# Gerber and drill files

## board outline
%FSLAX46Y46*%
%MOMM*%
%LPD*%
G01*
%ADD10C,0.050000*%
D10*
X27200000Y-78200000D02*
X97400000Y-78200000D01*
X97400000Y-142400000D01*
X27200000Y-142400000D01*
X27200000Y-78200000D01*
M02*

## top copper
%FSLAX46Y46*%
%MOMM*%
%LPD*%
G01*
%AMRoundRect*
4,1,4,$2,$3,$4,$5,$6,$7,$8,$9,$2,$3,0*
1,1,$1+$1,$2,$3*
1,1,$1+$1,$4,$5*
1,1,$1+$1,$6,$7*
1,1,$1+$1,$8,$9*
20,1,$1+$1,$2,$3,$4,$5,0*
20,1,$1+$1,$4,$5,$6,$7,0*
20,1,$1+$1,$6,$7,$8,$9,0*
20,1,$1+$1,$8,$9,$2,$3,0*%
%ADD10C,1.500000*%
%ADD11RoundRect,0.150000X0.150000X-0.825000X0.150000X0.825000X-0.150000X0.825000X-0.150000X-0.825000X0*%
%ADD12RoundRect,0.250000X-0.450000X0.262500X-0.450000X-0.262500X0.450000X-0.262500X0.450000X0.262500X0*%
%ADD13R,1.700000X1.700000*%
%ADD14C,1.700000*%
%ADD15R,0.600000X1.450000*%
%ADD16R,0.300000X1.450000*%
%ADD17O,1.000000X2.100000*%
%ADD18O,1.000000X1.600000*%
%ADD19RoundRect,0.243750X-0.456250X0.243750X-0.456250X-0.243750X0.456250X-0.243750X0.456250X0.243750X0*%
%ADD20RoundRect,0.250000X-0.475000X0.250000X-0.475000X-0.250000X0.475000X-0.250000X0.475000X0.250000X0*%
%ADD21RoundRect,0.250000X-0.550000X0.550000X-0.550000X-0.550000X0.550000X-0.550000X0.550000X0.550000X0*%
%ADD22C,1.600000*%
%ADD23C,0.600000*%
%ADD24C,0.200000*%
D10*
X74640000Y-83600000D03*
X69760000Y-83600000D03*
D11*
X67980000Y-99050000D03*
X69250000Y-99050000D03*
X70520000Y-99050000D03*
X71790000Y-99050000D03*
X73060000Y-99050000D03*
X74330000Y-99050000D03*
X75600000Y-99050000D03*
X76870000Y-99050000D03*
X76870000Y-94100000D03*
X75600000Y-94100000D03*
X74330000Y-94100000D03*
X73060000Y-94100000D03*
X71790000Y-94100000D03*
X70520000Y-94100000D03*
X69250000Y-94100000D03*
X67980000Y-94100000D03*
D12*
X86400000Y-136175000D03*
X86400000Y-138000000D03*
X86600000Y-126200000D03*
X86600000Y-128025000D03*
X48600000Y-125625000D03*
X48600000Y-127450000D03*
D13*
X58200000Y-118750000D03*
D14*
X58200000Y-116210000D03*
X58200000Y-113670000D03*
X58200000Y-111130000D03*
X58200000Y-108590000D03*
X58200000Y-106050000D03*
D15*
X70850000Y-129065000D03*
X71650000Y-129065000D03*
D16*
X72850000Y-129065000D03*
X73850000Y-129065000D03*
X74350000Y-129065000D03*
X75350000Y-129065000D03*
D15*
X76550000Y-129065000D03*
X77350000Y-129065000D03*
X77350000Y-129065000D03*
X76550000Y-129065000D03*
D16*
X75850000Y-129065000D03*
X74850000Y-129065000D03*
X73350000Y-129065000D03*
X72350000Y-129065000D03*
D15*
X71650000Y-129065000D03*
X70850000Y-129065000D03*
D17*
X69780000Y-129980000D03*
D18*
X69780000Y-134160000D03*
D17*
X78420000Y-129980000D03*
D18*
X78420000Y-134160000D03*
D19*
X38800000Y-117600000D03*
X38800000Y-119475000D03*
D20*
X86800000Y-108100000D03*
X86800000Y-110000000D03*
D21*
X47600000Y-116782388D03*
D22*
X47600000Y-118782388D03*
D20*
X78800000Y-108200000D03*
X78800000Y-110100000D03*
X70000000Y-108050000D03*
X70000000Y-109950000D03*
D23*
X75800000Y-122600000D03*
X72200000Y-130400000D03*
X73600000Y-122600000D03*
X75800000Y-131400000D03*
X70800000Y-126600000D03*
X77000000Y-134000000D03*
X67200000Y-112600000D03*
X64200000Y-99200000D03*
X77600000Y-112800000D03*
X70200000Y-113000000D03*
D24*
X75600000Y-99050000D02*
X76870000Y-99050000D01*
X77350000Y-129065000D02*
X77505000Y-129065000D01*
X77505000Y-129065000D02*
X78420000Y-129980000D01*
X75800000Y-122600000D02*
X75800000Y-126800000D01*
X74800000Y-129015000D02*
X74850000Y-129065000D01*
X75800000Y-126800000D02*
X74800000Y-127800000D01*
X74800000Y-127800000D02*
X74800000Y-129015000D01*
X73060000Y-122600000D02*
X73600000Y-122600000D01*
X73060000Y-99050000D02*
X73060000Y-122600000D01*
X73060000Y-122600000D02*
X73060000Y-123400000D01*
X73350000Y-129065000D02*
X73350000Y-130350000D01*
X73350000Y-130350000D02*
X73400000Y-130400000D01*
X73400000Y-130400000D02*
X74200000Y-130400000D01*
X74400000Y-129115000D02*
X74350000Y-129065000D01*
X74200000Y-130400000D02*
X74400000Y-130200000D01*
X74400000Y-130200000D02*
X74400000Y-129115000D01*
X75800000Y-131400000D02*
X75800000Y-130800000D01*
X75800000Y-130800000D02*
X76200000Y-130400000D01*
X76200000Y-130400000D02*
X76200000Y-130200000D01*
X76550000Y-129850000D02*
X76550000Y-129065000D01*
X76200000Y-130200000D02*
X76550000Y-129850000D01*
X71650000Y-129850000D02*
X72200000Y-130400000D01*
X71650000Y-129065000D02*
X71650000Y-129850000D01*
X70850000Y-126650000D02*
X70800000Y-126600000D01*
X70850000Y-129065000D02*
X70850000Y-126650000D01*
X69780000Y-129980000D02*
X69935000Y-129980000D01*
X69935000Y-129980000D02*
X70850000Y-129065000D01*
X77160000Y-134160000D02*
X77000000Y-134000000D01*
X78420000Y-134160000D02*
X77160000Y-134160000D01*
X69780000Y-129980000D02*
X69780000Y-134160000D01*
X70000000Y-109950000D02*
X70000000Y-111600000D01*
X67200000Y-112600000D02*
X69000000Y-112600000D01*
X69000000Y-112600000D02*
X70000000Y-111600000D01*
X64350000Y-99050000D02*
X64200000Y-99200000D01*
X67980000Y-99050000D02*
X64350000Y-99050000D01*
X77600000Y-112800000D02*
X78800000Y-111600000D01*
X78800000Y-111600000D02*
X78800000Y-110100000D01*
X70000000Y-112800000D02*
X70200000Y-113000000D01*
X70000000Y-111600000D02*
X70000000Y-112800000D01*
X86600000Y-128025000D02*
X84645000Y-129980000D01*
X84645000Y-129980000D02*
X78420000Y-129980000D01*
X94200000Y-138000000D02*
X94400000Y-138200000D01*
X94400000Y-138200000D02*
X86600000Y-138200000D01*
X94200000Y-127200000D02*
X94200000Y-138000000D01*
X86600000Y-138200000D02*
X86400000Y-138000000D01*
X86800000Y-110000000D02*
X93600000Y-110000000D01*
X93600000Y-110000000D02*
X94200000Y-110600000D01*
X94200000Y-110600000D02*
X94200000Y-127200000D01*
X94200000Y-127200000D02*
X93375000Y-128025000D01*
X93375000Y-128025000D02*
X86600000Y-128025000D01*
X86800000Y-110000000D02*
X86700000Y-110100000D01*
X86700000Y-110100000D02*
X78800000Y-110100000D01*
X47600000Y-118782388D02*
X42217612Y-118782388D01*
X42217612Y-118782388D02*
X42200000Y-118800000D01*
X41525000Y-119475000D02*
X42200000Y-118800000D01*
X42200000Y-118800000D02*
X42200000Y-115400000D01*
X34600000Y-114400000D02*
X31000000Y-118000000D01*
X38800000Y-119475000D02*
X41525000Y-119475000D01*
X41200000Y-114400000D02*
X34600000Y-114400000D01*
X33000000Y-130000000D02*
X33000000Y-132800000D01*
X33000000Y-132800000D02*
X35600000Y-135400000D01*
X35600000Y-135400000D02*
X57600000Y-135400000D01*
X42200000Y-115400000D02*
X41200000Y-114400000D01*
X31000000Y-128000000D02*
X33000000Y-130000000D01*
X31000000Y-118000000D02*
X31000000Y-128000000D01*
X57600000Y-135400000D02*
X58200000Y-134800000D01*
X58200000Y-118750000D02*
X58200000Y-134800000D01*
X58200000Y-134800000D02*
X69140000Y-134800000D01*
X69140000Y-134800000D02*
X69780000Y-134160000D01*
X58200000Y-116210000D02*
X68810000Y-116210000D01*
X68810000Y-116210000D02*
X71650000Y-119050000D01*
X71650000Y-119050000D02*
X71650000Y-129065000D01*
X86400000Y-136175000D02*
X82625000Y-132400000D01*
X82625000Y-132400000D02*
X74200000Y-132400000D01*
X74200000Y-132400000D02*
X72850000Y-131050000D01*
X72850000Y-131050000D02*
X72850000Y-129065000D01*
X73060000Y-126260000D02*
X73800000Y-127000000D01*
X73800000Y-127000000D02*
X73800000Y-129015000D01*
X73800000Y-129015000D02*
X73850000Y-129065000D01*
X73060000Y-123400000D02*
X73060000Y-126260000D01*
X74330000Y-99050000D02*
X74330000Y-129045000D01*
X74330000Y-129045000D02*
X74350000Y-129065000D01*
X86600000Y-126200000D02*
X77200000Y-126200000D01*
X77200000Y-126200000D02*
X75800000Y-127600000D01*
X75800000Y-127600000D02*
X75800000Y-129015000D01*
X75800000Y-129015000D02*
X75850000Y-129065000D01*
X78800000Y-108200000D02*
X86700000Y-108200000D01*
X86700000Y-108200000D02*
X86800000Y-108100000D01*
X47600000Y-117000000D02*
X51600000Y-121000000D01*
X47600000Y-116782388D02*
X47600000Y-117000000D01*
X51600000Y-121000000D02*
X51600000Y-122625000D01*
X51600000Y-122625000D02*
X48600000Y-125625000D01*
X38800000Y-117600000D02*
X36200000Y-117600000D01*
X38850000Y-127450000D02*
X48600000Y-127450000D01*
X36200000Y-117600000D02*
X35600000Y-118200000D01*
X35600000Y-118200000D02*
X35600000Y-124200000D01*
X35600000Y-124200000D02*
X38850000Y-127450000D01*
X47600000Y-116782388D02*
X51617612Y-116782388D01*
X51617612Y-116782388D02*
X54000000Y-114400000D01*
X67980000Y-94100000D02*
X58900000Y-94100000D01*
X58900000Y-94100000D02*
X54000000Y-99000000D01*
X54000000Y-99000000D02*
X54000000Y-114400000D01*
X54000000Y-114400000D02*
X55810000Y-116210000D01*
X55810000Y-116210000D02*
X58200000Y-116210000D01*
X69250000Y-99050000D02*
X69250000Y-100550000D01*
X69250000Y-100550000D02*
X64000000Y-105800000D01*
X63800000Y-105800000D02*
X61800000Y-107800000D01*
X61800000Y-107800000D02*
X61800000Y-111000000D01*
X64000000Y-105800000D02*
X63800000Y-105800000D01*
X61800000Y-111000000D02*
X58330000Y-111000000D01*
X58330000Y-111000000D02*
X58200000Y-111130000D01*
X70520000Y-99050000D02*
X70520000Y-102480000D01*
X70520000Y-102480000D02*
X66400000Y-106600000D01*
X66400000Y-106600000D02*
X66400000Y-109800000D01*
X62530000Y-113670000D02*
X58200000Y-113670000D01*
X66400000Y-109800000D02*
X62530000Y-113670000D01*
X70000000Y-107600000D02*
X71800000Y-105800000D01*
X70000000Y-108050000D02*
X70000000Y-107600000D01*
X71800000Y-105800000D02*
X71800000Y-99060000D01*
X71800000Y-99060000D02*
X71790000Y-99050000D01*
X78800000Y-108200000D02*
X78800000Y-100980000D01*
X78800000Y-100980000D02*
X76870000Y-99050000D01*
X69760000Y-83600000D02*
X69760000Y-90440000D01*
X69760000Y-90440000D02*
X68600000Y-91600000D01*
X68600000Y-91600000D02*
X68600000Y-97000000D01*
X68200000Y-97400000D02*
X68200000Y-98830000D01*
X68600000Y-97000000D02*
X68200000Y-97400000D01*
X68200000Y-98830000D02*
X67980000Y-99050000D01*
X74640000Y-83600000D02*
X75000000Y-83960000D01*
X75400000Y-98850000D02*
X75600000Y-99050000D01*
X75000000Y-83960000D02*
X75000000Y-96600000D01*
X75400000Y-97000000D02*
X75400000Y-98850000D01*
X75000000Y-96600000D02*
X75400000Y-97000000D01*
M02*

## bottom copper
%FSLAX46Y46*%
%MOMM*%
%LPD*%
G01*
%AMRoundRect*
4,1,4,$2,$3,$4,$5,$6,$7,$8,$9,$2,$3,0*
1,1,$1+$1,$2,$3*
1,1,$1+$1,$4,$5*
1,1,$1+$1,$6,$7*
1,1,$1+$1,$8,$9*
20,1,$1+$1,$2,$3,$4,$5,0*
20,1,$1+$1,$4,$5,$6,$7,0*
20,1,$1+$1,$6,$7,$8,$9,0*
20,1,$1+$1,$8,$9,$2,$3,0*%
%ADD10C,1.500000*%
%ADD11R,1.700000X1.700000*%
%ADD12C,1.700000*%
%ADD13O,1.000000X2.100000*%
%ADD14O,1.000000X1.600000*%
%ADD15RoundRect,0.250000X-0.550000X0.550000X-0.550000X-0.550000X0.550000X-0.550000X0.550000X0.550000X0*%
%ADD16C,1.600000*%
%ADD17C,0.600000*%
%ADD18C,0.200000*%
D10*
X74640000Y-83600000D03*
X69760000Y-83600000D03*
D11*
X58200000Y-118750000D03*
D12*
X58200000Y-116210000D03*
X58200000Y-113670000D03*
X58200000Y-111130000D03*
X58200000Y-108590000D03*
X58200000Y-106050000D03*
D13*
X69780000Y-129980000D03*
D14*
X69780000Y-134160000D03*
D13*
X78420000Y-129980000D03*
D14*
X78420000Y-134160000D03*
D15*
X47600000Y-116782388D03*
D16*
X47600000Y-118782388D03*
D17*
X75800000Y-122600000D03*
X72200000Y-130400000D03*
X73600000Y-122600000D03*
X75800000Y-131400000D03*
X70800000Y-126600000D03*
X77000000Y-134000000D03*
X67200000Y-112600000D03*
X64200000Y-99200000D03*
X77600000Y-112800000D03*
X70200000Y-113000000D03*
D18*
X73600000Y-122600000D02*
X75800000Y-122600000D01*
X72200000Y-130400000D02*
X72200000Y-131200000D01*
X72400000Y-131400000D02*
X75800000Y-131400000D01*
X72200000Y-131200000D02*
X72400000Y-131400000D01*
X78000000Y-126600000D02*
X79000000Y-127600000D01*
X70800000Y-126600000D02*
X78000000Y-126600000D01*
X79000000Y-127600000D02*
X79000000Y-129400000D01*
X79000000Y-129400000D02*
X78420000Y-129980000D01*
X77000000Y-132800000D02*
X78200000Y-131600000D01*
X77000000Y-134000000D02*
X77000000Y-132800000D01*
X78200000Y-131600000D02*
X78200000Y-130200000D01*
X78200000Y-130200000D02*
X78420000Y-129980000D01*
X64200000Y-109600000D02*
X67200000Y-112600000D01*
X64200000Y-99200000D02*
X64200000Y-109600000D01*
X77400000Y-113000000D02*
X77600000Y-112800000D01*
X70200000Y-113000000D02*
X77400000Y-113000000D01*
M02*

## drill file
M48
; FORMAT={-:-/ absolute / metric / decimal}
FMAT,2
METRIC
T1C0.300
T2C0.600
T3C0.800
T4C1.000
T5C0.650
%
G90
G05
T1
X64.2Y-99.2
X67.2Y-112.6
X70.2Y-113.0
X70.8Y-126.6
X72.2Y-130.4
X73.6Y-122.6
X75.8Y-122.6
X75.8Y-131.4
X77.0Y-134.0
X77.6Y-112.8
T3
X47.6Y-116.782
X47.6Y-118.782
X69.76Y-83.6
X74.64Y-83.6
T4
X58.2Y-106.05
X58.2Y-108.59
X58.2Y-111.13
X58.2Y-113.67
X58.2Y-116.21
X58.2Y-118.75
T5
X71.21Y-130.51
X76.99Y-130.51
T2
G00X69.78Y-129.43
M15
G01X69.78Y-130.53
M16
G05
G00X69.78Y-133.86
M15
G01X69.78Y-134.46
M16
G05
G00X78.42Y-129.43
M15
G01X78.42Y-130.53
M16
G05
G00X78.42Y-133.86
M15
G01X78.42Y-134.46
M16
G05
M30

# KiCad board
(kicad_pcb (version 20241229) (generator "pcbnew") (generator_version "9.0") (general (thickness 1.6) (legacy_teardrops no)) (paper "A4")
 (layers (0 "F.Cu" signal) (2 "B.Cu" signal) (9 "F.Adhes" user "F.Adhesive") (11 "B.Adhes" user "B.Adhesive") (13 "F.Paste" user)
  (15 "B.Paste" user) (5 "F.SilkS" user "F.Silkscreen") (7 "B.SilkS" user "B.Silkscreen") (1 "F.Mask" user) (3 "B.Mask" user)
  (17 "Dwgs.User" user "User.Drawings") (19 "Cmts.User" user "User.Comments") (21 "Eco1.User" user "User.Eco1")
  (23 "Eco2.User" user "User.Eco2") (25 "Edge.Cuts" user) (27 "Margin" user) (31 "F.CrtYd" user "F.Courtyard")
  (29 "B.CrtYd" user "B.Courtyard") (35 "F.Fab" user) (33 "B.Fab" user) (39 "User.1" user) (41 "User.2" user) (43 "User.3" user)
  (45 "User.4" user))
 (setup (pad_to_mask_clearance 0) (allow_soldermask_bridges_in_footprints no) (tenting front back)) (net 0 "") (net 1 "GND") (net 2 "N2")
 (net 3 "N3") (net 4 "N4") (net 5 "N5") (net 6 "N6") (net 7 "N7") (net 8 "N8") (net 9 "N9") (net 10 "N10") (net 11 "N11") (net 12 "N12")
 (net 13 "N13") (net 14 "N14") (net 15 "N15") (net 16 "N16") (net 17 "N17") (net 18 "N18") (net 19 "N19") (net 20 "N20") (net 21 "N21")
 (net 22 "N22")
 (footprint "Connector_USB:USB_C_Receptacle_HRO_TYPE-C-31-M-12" (layer "F.Cu") (at 74.1 133.11)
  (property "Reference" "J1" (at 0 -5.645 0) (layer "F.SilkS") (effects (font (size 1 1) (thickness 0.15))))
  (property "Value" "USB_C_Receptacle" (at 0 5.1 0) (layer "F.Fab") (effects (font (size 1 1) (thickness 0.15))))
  (pad "" np_thru_hole circle (at -2.89 -2.6) (size 0.65 0.65) (drill 0.65) (layers "*.Cu" "*.Mask"))
  (pad "" np_thru_hole circle (at 2.89 -2.6) (size 0.65 0.65) (drill 0.65) (layers "*.Cu" "*.Mask"))
  (pad "A1" smd rect (at -3.25 -4.045) (size 0.6 1.45) (layers "F.Cu" "F.Mask" "F.Paste") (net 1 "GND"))
  (pad "A4" smd rect (at -2.45 -4.045) (size 0.6 1.45) (layers "F.Cu" "F.Mask" "F.Paste") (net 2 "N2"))
  (pad "A5" smd rect (at -1.25 -4.045) (size 0.3 1.45) (layers "F.Cu" "F.Mask" "F.Paste") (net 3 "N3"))
  (pad "A6" smd rect (at -0.25 -4.045) (size 0.3 1.45) (layers "F.Cu" "F.Mask" "F.Paste") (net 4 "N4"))
  (pad "A7" smd rect (at 0.25 -4.045) (size 0.3 1.45) (layers "F.Cu" "F.Mask" "F.Paste") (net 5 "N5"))
  (pad "A8" smd rect (at 1.25 -4.045) (size 0.3 1.45) (layers "F.Cu" "F.Mask" "F.Paste") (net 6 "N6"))
  (pad "A9" smd rect (at 2.45 -4.045) (size 0.6 1.45) (layers "F.Cu" "F.Mask" "F.Paste") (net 2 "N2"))
  (pad "A12" smd rect (at 3.25 -4.045) (size 0.6 1.45) (layers "F.Cu" "F.Mask" "F.Paste") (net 1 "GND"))
  (pad "B1" smd rect (at 3.25 -4.045) (size 0.6 1.45) (layers "F.Cu" "F.Mask" "F.Paste") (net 1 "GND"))
  (pad "B4" smd rect (at 2.45 -4.045) (size 0.6 1.45) (layers "F.Cu" "F.Mask" "F.Paste") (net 2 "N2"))
  (pad "B5" smd rect (at 1.75 -4.045) (size 0.3 1.45) (layers "F.Cu" "F.Mask" "F.Paste") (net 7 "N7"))
  (pad "B6" smd rect (at 0.75 -4.045) (size 0.3 1.45) (layers "F.Cu" "F.Mask" "F.Paste") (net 4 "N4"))
  (pad "B7" smd rect (at -0.75 -4.045) (size 0.3 1.45) (layers "F.Cu" "F.Mask" "F.Paste") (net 5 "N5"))
  (pad "B8" smd rect (at -1.75 -4.045) (size 0.3 1.45) (layers "F.Cu" "F.Mask" "F.Paste") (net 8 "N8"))
  (pad "B9" smd rect (at -2.45 -4.045) (size 0.6 1.45) (layers "F.Cu" "F.Mask" "F.Paste") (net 2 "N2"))
  (pad "B12" smd rect (at -3.25 -4.045) (size 0.6 1.45) (layers "F.Cu" "F.Mask" "F.Paste") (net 1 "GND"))
  (pad "S1" thru_hole oval (at -4.32 -3.13) (size 1 2.1) (drill oval 0.6 1.7) (layers "*.Cu" "*.Mask") (remove_unused_layers no)
   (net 1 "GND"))
  (pad "S1" thru_hole oval (at -4.32 1.05) (size 1 1.6) (drill oval 0.6 1.2) (layers "*.Cu" "*.Mask") (remove_unused_layers no)
   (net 1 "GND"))
  (pad "S1" thru_hole oval (at 4.32 -3.13) (size 1 2.1) (drill oval 0.6 1.7) (layers "*.Cu" "*.Mask") (remove_unused_layers no)
   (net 1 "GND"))
  (pad "S1" thru_hole oval (at 4.32 1.05) (size 1 1.6) (drill oval 0.6 1.2) (layers "*.Cu" "*.Mask") (remove_unused_layers no) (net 1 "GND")))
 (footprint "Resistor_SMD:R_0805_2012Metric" (layer "F.Cu") (at 86.6 127.1125 -90)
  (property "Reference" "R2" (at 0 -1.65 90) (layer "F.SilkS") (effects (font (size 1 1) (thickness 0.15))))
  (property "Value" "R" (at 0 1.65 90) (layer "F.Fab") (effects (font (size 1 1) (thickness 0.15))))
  (pad "1" smd roundrect (at -0.9125 0 270) (size 1.025 1.4) (layers "F.Cu" "F.Mask" "F.Paste") (roundrect_rratio 0.243902) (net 7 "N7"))
  (pad "2" smd roundrect (at 0.9125 0 270) (size 1.025 1.4) (layers "F.Cu" "F.Mask" "F.Paste") (roundrect_rratio 0.243902) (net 1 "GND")))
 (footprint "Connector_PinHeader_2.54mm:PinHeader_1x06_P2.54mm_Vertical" (layer "F.Cu") (at 58.2 118.75 180)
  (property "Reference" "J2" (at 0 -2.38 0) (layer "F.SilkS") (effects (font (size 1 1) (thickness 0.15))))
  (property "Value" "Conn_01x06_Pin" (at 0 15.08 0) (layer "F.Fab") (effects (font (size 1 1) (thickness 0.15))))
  (pad "1" thru_hole rect (at 0 0 180) (size 1.7 1.7) (drill 1) (layers "*.Cu" "*.Mask") (remove_unused_layers no) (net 1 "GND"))
  (pad "2" thru_hole circle (at 0 2.54 180) (size 1.7 1.7) (drill 1) (layers "*.Cu" "*.Mask") (remove_unused_layers no) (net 2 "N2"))
  (pad "3" thru_hole circle (at 0 5.08 180) (size 1.7 1.7) (drill 1) (layers "*.Cu" "*.Mask") (remove_unused_layers no) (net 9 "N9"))
  (pad "4" thru_hole circle (at 0 7.62 180) (size 1.7 1.7) (drill 1) (layers "*.Cu" "*.Mask") (remove_unused_layers no) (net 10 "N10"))
  (pad "5" thru_hole circle (at 0 10.16 180) (size 1.7 1.7) (drill 1) (layers "*.Cu" "*.Mask") (remove_unused_layers no) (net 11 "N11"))
  (pad "6" thru_hole circle (at 0 12.7 180) (size 1.7 1.7) (drill 1) (layers "*.Cu" "*.Mask") (remove_unused_layers no) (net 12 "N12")))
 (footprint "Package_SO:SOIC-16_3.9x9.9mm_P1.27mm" (layer "F.Cu") (at 72.425 96.575 90)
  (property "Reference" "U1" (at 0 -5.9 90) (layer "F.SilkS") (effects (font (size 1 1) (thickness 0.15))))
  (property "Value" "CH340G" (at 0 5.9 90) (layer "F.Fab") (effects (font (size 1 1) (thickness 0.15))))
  (pad "1" smd roundrect (at -2.475 -4.445 90) (size 1.95 0.6) (layers "F.Cu" "F.Mask" "F.Paste") (roundrect_rratio 0.25) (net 1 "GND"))
  (pad "2" smd roundrect (at -2.475 -3.175 90) (size 1.95 0.6) (layers "F.Cu" "F.Mask" "F.Paste") (roundrect_rratio 0.25) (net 10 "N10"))
  (pad "3" smd roundrect (at -2.475 -1.905 90) (size 1.95 0.6) (layers "F.Cu" "F.Mask" "F.Paste") (roundrect_rratio 0.25) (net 9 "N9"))
  (pad "4" smd roundrect (at -2.475 -0.635 90) (size 1.95 0.6) (layers "F.Cu" "F.Mask" "F.Paste") (roundrect_rratio 0.25) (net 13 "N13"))
  (pad "5" smd roundrect (at -2.475 0.635 90) (size 1.95 0.6) (layers "F.Cu" "F.Mask" "F.Paste") (roundrect_rratio 0.25) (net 4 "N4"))
  (pad "6" smd roundrect (at -2.475 1.905 90) (size 1.95 0.6) (layers "F.Cu" "F.Mask" "F.Paste") (roundrect_rratio 0.25) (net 5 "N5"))
  (pad "7" smd roundrect (at -2.475 3.175 90) (size 1.95 0.6) (layers "F.Cu" "F.Mask" "F.Paste") (roundrect_rratio 0.25) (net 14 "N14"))
  (pad "8" smd roundrect (at -2.475 4.445 90) (size 1.95 0.6) (layers "F.Cu" "F.Mask" "F.Paste") (roundrect_rratio 0.25) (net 14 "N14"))
  (pad "9" smd roundrect (at 2.475 4.445 90) (size 1.95 0.6) (layers "F.Cu" "F.Mask" "F.Paste") (roundrect_rratio 0.25) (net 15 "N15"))
  (pad "10" smd roundrect (at 2.475 3.175 90) (size 1.95 0.6) (layers "F.Cu" "F.Mask" "F.Paste") (roundrect_rratio 0.25) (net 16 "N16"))
  (pad "11" smd roundrect (at 2.475 1.905 90) (size 1.95 0.6) (layers "F.Cu" "F.Mask" "F.Paste") (roundrect_rratio 0.25) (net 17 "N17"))
  (pad "12" smd roundrect (at 2.475 0.635 90) (size 1.95 0.6) (layers "F.Cu" "F.Mask" "F.Paste") (roundrect_rratio 0.25) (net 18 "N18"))
  (pad "13" smd roundrect (at 2.475 -0.635 90) (size 1.95 0.6) (layers "F.Cu" "F.Mask" "F.Paste") (roundrect_rratio 0.25) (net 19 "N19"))
  (pad "14" smd roundrect (at 2.475 -1.905 90) (size 1.95 0.6) (layers "F.Cu" "F.Mask" "F.Paste") (roundrect_rratio 0.25) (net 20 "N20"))
  (pad "15" smd roundrect (at 2.475 -3.175 90) (size 1.95 0.6) (layers "F.Cu" "F.Mask" "F.Paste") (roundrect_rratio 0.25) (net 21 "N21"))
  (pad "16" smd roundrect (at 2.475 -4.445 90) (size 1.95 0.6) (layers "F.Cu" "F.Mask" "F.Paste") (roundrect_rratio 0.25) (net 2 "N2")))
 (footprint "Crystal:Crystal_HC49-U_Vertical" (layer "F.Cu") (at 74.64 83.6 180)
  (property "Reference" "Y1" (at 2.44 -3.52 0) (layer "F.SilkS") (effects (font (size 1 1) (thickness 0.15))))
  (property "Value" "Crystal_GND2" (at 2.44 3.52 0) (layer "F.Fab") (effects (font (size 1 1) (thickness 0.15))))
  (pad "1" thru_hole circle (at 0 0 180) (size 1.5 1.5) (drill 0.8) (layers "*.Cu" "*.Mask") (remove_unused_layers no) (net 14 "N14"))
  (pad "2" thru_hole circle (at 4.88 0 180) (size 1.5 1.5) (drill 0.8) (layers "*.Cu" "*.Mask") (remove_unused_layers no) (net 1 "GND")))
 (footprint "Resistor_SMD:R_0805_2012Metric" (layer "F.Cu") (at 86.4 137.0875 -90)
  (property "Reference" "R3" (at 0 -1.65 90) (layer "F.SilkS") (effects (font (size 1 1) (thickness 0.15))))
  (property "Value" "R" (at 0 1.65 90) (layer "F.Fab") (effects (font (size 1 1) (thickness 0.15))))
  (pad "1" smd roundrect (at -0.9125 0 270) (size 1.025 1.4) (layers "F.Cu" "F.Mask" "F.Paste") (roundrect_rratio 0.243902) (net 3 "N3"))
  (pad "2" smd roundrect (at 0.9125 0 270) (size 1.025 1.4) (layers "F.Cu" "F.Mask" "F.Paste") (roundrect_rratio 0.243902) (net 1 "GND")))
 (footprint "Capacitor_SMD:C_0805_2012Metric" (layer "F.Cu") (at 70 109 -90)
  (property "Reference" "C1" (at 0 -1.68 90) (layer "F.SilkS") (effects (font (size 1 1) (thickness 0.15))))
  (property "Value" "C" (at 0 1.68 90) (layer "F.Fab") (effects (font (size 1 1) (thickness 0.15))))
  (pad "1" smd roundrect (at -0.95 0 270) (size 1 1.45) (layers "F.Cu" "F.Mask" "F.Paste") (roundrect_rratio 0.25) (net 13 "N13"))
  (pad "2" smd roundrect (at 0.95 0 270) (size 1 1.45) (layers "F.Cu" "F.Mask" "F.Paste") (roundrect_rratio 0.25) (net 1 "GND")))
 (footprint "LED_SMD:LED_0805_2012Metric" (layer "F.Cu") (at 38.8 118.5375 -90)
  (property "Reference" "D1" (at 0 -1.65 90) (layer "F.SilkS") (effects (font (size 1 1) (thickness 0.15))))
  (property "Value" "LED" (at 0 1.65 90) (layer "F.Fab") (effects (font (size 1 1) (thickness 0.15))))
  (pad "1" smd roundrect (at -0.9375 0 270) (size 0.975 1.4) (layers "F.Cu" "F.Mask" "F.Paste") (roundrect_rratio 0.25) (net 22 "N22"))
  (pad "2" smd roundrect (at 0.9375 0 270) (size 0.975 1.4) (layers "F.Cu" "F.Mask" "F.Paste") (roundrect_rratio 0.25) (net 1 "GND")))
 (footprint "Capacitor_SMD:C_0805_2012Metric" (layer "F.Cu") (at 86.8 109.05 -90)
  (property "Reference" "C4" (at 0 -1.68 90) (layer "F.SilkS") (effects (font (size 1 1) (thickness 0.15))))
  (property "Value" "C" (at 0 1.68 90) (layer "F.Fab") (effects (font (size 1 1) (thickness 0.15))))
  (pad "1" smd roundrect (at -0.95 0 270) (size 1 1.45) (layers "F.Cu" "F.Mask" "F.Paste") (roundrect_rratio 0.25) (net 14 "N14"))
  (pad "2" smd roundrect (at 0.95 0 270) (size 1 1.45) (layers "F.Cu" "F.Mask" "F.Paste") (roundrect_rratio 0.25) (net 1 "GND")))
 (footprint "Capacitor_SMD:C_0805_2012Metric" (layer "F.Cu") (at 78.8 109.15 -90)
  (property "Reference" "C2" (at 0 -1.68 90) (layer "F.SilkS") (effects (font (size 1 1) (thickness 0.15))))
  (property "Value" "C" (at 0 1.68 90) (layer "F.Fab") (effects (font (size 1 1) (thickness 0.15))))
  (pad "1" smd roundrect (at -0.95 0 270) (size 1 1.45) (layers "F.Cu" "F.Mask" "F.Paste") (roundrect_rratio 0.25) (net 14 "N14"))
  (pad "2" smd roundrect (at 0.95 0 270) (size 1 1.45) (layers "F.Cu" "F.Mask" "F.Paste") (roundrect_rratio 0.25) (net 1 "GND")))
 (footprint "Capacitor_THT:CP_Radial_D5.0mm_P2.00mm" (layer "F.Cu") (at 47.6 116.782388 -90)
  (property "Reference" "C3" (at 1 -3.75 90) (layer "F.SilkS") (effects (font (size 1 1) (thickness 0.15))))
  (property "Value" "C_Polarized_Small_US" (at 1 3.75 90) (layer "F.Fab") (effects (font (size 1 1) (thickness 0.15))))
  (pad "1" thru_hole roundrect (at 0 0 270) (size 1.6 1.6) (drill 0.8) (layers "*.Cu" "*.Mask") (remove_unused_layers no)
   (roundrect_rratio 0.15625) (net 2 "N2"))
  (pad "2" thru_hole circle (at 2 0 270) (size 1.6 1.6) (drill 0.8) (layers "*.Cu" "*.Mask") (remove_unused_layers no) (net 1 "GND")))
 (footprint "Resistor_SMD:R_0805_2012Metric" (layer "F.Cu") (at 48.6 126.5375 -90)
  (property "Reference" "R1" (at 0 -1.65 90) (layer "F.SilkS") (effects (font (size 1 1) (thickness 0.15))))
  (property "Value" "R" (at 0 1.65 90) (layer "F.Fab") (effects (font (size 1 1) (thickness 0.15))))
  (pad "1" smd roundrect (at -0.9125 0 270) (size 1.025 1.4) (layers "F.Cu" "F.Mask" "F.Paste") (roundrect_rratio 0.243902) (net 2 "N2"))
  (pad "2" smd roundrect (at 0.9125 0 270) (size 1.025 1.4) (layers "F.Cu" "F.Mask" "F.Paste") (roundrect_rratio 0.243902) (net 22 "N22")))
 (gr_rect (start 27.2 78.2) (end 97.4 142.4) (stroke (width 0.05) (type default)) (fill no) (layer "Edge.Cuts"))
 (segment (start 86.8 110) (end 93.6 110) (width 0.2) (layer "F.Cu") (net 1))
 (segment (start 86.6 138.2) (end 86.4 138) (width 0.2) (layer "F.Cu") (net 1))
 (segment (start 58.2 118.75) (end 58.2 134.8) (width 0.2) (layer "F.Cu") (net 1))
 (segment (start 77.16 134.16) (end 77 134) (width 0.2) (layer "F.Cu") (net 1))
 (segment (start 67.2 112.6) (end 69 112.6) (width 0.2) (layer "F.Cu") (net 1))
 (segment (start 94.2 127.2) (end 93.375 128.025) (width 0.2) (layer "F.Cu") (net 1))
 (segment (start 69.76 83.6) (end 69.76 90.44) (width 0.2) (layer "F.Cu") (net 1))
 (segment (start 69.76 90.44) (end 68.6 91.6) (width 0.2) (layer "F.Cu") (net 1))
 (segment (start 64.35 99.05) (end 64.2 99.2) (width 0.2) (layer "F.Cu") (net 1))
 (segment (start 77.6 112.8) (end 78.8 111.6) (width 0.2) (layer "F.Cu") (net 1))
 (segment (start 33 130) (end 33 132.8) (width 0.2) (layer "F.Cu") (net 1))
 (segment (start 78.8 111.6) (end 78.8 110.1) (width 0.2) (layer "F.Cu") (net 1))
 (segment (start 77.35 129.065) (end 77.505 129.065) (width 0.2) (layer "F.Cu") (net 1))
 (segment (start 86.8 110) (end 86.7 110.1) (width 0.2) (layer "F.Cu") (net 1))
 (segment (start 33 132.8) (end 35.6 135.4) (width 0.2) (layer "F.Cu") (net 1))
 (segment (start 38.8 119.475) (end 41.525 119.475) (width 0.2) (layer "F.Cu") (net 1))
 (segment (start 34.6 114.4) (end 31 118) (width 0.2) (layer "F.Cu") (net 1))
 (segment (start 69.78 129.98) (end 69.78 134.16) (width 0.2) (layer "F.Cu") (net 1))
 (segment (start 67.98 99.05) (end 64.35 99.05) (width 0.2) (layer "F.Cu") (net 1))
 (segment (start 70 109.95) (end 70 111.6) (width 0.2) (layer "F.Cu") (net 1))
 (segment (start 69.935 129.98) (end 70.85 129.065) (width 0.2) (layer "F.Cu") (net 1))
 (segment (start 42.2 115.4) (end 41.2 114.4) (width 0.2) (layer "F.Cu") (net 1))
 (segment (start 69.14 134.8) (end 69.78 134.16) (width 0.2) (layer "F.Cu") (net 1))
 (segment (start 77.505 129.065) (end 78.42 129.98) (width 0.2) (layer "F.Cu") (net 1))
 (segment (start 86.7 110.1) (end 78.8 110.1) (width 0.2) (layer "F.Cu") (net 1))
 (segment (start 93.375 128.025) (end 86.6 128.025) (width 0.2) (layer "F.Cu") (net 1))
 (segment (start 58.2 134.8) (end 69.14 134.8) (width 0.2) (layer "F.Cu") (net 1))
 (segment (start 35.6 135.4) (end 57.6 135.4) (width 0.2) (layer "F.Cu") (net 1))
 (segment (start 68.2 98.83) (end 67.98 99.05) (width 0.2) (layer "F.Cu") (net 1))
 (segment (start 68.2 97.4) (end 68.2 98.83) (width 0.2) (layer "F.Cu") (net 1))
 (segment (start 70 111.6) (end 70 112.8) (width 0.2) (layer "F.Cu") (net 1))
 (segment (start 94.2 110.6) (end 94.2 127.2) (width 0.2) (layer "F.Cu") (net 1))
 (segment (start 57.6 135.4) (end 58.2 134.8) (width 0.2) (layer "F.Cu") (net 1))
 (segment (start 68.6 97) (end 68.2 97.4) (width 0.2) (layer "F.Cu") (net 1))
 (segment (start 68.6 91.6) (end 68.6 97) (width 0.2) (layer "F.Cu") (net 1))
 (segment (start 93.6 110) (end 94.2 110.6) (width 0.2) (layer "F.Cu") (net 1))
 (segment (start 70.85 129.065) (end 70.85 126.65) (width 0.2) (layer "F.Cu") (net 1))
 (segment (start 84.645 129.98) (end 78.42 129.98) (width 0.2) (layer "F.Cu") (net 1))
 (segment (start 31 128) (end 33 130) (width 0.2) (layer "F.Cu") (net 1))
 (segment (start 42.2 118.8) (end 42.2 115.4) (width 0.2) (layer "F.Cu") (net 1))
 (segment (start 94.2 138) (end 94.4 138.2) (width 0.2) (layer "F.Cu") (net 1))
 (segment (start 70 112.8) (end 70.2 113) (width 0.2) (layer "F.Cu") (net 1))
 (segment (start 70.85 126.65) (end 70.8 126.6) (width 0.2) (layer "F.Cu") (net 1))
 (segment (start 41.525 119.475) (end 42.2 118.8) (width 0.2) (layer "F.Cu") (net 1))
 (segment (start 86.6 128.025) (end 84.645 129.98) (width 0.2) (layer "F.Cu") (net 1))
 (segment (start 94.4 138.2) (end 86.6 138.2) (width 0.2) (layer "F.Cu") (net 1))
 (segment (start 94.2 127.2) (end 94.2 138) (width 0.2) (layer "F.Cu") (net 1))
 (segment (start 31 118) (end 31 128) (width 0.2) (layer "F.Cu") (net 1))
 (segment (start 42.217612 118.782388) (end 42.2 118.8) (width 0.2) (layer "F.Cu") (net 1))
 (segment (start 69 112.6) (end 70 111.6) (width 0.2) (layer "F.Cu") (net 1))
 (segment (start 47.6 118.782388) (end 42.217612 118.782388) (width 0.2) (layer "F.Cu") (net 1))
 (segment (start 69.78 129.98) (end 69.935 129.98) (width 0.2) (layer "F.Cu") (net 1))
 (segment (start 78.42 134.16) (end 77.16 134.16) (width 0.2) (layer "F.Cu") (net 1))
 (segment (start 41.2 114.4) (end 34.6 114.4) (width 0.2) (layer "F.Cu") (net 1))
 (via (at 67.2 112.6) (size 0.6) (drill 0.3) (layers "F.Cu" "B.Cu") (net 1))
 (via (at 70.2 113) (size 0.6) (drill 0.3) (layers "F.Cu" "B.Cu") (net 1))
 (via (at 77 134) (size 0.6) (drill 0.3) (layers "F.Cu" "B.Cu") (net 1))
 (via (at 64.2 99.2) (size 0.6) (drill 0.3) (layers "F.Cu" "B.Cu") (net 1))
 (via (at 77.6 112.8) (size 0.6) (drill 0.3) (layers "F.Cu" "B.Cu") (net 1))
 (via (at 70.8 126.6) (size 0.6) (drill 0.3) (layers "F.Cu" "B.Cu") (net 1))
 (segment (start 77.4 113) (end 77.6 112.8) (width 0.2) (layer "B.Cu") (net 1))
 (segment (start 70.8 126.6) (end 78 126.6) (width 0.2) (layer "B.Cu") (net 1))
 (segment (start 77 132.8) (end 78.2 131.6) (width 0.2) (layer "B.Cu") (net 1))
 (segment (start 64.2 99.2) (end 64.2 109.6) (width 0.2) (layer "B.Cu") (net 1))
 (segment (start 79 129.4) (end 78.42 129.98) (width 0.2) (layer "B.Cu") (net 1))
 (segment (start 79 127.6) (end 79 129.4) (width 0.2) (layer "B.Cu") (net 1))
 (segment (start 78.2 130.2) (end 78.42 129.98) (width 0.2) (layer "B.Cu") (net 1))
 (segment (start 70.2 113) (end 77.4 113) (width 0.2) (layer "B.Cu") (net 1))
 (segment (start 78 126.6) (end 79 127.6) (width 0.2) (layer "B.Cu") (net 1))
 (segment (start 77 134) (end 77 132.8) (width 0.2) (layer "B.Cu") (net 1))
 (segment (start 78.2 131.6) (end 78.2 130.2) (width 0.2) (layer "B.Cu") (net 1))
 (segment (start 64.2 109.6) (end 67.2 112.6) (width 0.2) (layer "B.Cu") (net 1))
 (segment (start 71.8 99.06) (end 71.79 99.05) (width 0.2) (layer "F.Cu") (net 13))
 (segment (start 70 107.6) (end 71.8 105.8) (width 0.2) (layer "F.Cu") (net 13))
 (segment (start 71.8 105.8) (end 71.8 99.06) (width 0.2) (layer "F.Cu") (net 13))
 (segment (start 70 108.05) (end 70 107.6) (width 0.2) (layer "F.Cu") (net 13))
 (segment (start 75 96.6) (end 75.4 97) (width 0.2) (layer "F.Cu") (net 14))
 (segment (start 75.4 98.85) (end 75.6 99.05) (width 0.2) (layer "F.Cu") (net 14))
 (segment (start 78.8 108.2) (end 86.7 108.2) (width 0.2) (layer "F.Cu") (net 14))
 (segment (start 75.4 97) (end 75.4 98.85) (width 0.2) (layer "F.Cu") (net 14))
 (segment (start 74.64 83.6) (end 75 83.96) (width 0.2) (layer "F.Cu") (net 14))
 (segment (start 78.8 100.98) (end 76.87 99.05) (width 0.2) (layer "F.Cu") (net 14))
 (segment (start 75 83.96) (end 75 96.6) (width 0.2) (layer "F.Cu") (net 14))
 (segment (start 75.6 99.05) (end 76.87 99.05) (width 0.2) (layer "F.Cu") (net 14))
 (segment (start 86.7 108.2) (end 86.8 108.1) (width 0.2) (layer "F.Cu") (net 14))
 (segment (start 78.8 108.2) (end 78.8 100.98) (width 0.2) (layer "F.Cu") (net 14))
 (segment (start 67.98 94.1) (end 58.9 94.1) (width 0.2) (layer "F.Cu") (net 2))
 (segment (start 71.65 129.85) (end 72.2 130.4) (width 0.2) (layer "F.Cu") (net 2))
 (segment (start 71.65 129.065) (end 71.65 129.85) (width 0.2) (layer "F.Cu") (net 2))
 (segment (start 54 114.4) (end 55.81 116.21) (width 0.2) (layer "F.Cu") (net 2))
 (segment (start 75.8 131.4) (end 75.8 130.8) (width 0.2) (layer "F.Cu") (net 2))
 (segment (start 58.2 116.21) (end 68.81 116.21) (width 0.2) (layer "F.Cu") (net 2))
 (segment (start 58.9 94.1) (end 54 99) (width 0.2) (layer "F.Cu") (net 2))
 (segment (start 47.6 116.782388) (end 51.617612 116.782388) (width 0.2) (layer "F.Cu") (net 2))
 (segment (start 76.2 130.2) (end 76.55 129.85) (width 0.2) (layer "F.Cu") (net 2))
 (segment (start 51.6 121) (end 51.6 122.625) (width 0.2) (layer "F.Cu") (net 2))
 (segment (start 75.8 130.8) (end 76.2 130.4) (width 0.2) (layer "F.Cu") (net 2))
 (segment (start 71.65 119.05) (end 71.65 129.065) (width 0.2) (layer "F.Cu") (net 2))
 (segment (start 54 99) (end 54 114.4) (width 0.2) (layer "F.Cu") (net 2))
 (segment (start 51.6 122.625) (end 48.6 125.625) (width 0.2) (layer "F.Cu") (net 2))
 (segment (start 76.55 129.85) (end 76.55 129.065) (width 0.2) (layer "F.Cu") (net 2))
 (segment (start 68.81 116.21) (end 71.65 119.05) (width 0.2) (layer "F.Cu") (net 2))
 (segment (start 47.6 116.782388) (end 47.6 117) (width 0.2) (layer "F.Cu") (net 2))
 (segment (start 55.81 116.21) (end 58.2 116.21) (width 0.2) (layer "F.Cu") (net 2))
 (segment (start 47.6 117) (end 51.6 121) (width 0.2) (layer "F.Cu") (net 2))
 (segment (start 51.617612 116.782388) (end 54 114.4) (width 0.2) (layer "F.Cu") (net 2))
 (segment (start 76.2 130.4) (end 76.2 130.2) (width 0.2) (layer "F.Cu") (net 2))
 (via (at 72.2 130.4) (size 0.6) (drill 0.3) (layers "F.Cu" "B.Cu") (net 2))
 (via (at 75.8 131.4) (size 0.6) (drill 0.3) (layers "F.Cu" "B.Cu") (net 2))
 (segment (start 72.2 131.2) (end 72.4 131.4) (width 0.2) (layer "B.Cu") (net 2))
 (segment (start 72.2 130.4) (end 72.2 131.2) (width 0.2) (layer "B.Cu") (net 2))
 (segment (start 72.4 131.4) (end 75.8 131.4) (width 0.2) (layer "B.Cu") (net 2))
 (segment (start 36.2 117.6) (end 35.6 118.2) (width 0.2) (layer "F.Cu") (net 22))
 (segment (start 35.6 118.2) (end 35.6 124.2) (width 0.2) (layer "F.Cu") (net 22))
 (segment (start 38.8 117.6) (end 36.2 117.6) (width 0.2) (layer "F.Cu") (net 22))
 (segment (start 35.6 124.2) (end 38.85 127.45) (width 0.2) (layer "F.Cu") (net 22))
 (segment (start 38.85 127.45) (end 48.6 127.45) (width 0.2) (layer "F.Cu") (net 22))
 (segment (start 74.33 129.045) (end 74.35 129.065) (width 0.2) (layer "F.Cu") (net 5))
 (segment (start 74.33 99.05) (end 74.33 129.045) (width 0.2) (layer "F.Cu") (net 5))
 (segment (start 73.4 130.4) (end 74.2 130.4) (width 0.2) (layer "F.Cu") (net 5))
 (segment (start 74.4 129.115) (end 74.35 129.065) (width 0.2) (layer "F.Cu") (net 5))
 (segment (start 73.35 130.35) (end 73.4 130.4) (width 0.2) (layer "F.Cu") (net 5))
 (segment (start 73.35 129.065) (end 73.35 130.35) (width 0.2) (layer "F.Cu") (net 5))
 (segment (start 74.4 130.2) (end 74.4 129.115) (width 0.2) (layer "F.Cu") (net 5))
 (segment (start 74.2 130.4) (end 74.4 130.2) (width 0.2) (layer "F.Cu") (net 5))
 (segment (start 73.8 127) (end 73.8 129.015) (width 0.2) (layer "F.Cu") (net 4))
 (segment (start 75.8 122.6) (end 75.8 126.8) (width 0.2) (layer "F.Cu") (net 4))
 (segment (start 74.8 129.015) (end 74.85 129.065) (width 0.2) (layer "F.Cu") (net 4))
 (segment (start 73.06 122.6) (end 73.6 122.6) (width 0.2) (layer "F.Cu") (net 4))
 (segment (start 73.06 126.26) (end 73.8 127) (width 0.2) (layer "F.Cu") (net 4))
 (segment (start 75.8 126.8) (end 74.8 127.8) (width 0.2) (layer "F.Cu") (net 4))
 (segment (start 74.8 127.8) (end 74.8 129.015) (width 0.2) (layer "F.Cu") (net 4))
 (segment (start 73.06 122.6) (end 73.06 123.4) (width 0.2) (layer "F.Cu") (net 4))
 (segment (start 73.8 129.015) (end 73.85 129.065) (width 0.2) (layer "F.Cu") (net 4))
 (segment (start 73.06 99.05) (end 73.06 122.6) (width 0.2) (layer "F.Cu") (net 4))
 (segment (start 73.06 123.4) (end 73.06 126.26) (width 0.2) (layer "F.Cu") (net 4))
 (via (at 73.6 122.6) (size 0.6) (drill 0.3) (layers "F.Cu" "B.Cu") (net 4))
 (via (at 75.8 122.6) (size 0.6) (drill 0.3) (layers "F.Cu" "B.Cu") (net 4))
 (segment (start 73.6 122.6) (end 75.8 122.6) (width 0.2) (layer "B.Cu") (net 4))
 (segment (start 75.8 129.015) (end 75.85 129.065) (width 0.2) (layer "F.Cu") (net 7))
 (segment (start 75.8 127.6) (end 75.8 129.015) (width 0.2) (layer "F.Cu") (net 7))
 (segment (start 77.2 126.2) (end 75.8 127.6) (width 0.2) (layer "F.Cu") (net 7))
 (segment (start 86.6 126.2) (end 77.2 126.2) (width 0.2) (layer "F.Cu") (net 7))
 (segment (start 74.2 132.4) (end 72.85 131.05) (width 0.2) (layer "F.Cu") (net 3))
 (segment (start 72.85 131.05) (end 72.85 129.065) (width 0.2) (layer "F.Cu") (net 3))
 (segment (start 86.4 136.175) (end 82.625 132.4) (width 0.2) (layer "F.Cu") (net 3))
 (segment (start 82.625 132.4) (end 74.2 132.4) (width 0.2) (layer "F.Cu") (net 3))
 (segment (start 64 105.8) (end 63.8 105.8) (width 0.2) (layer "F.Cu") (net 10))
 (segment (start 69.25 99.05) (end 69.25 100.55) (width 0.2) (layer "F.Cu") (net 10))
 (segment (start 61.8 107.8) (end 61.8 111) (width 0.2) (layer "F.Cu") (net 10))
 (segment (start 69.25 100.55) (end 64 105.8) (width 0.2) (layer "F.Cu") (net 10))
 (segment (start 58.33 111) (end 58.2 111.13) (width 0.2) (layer "F.Cu") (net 10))
 (segment (start 61.8 111) (end 58.33 111) (width 0.2) (layer "F.Cu") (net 10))
 (segment (start 63.8 105.8) (end 61.8 107.8) (width 0.2) (layer "F.Cu") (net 10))
 (segment (start 66.4 106.6) (end 66.4 109.8) (width 0.2) (layer "F.Cu") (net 9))
 (segment (start 66.4 109.8) (end 62.53 113.67) (width 0.2) (layer "F.Cu") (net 9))
 (segment (start 70.52 99.05) (end 70.52 102.48) (width 0.2) (layer "F.Cu") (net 9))
 (segment (start 70.52 102.48) (end 66.4 106.6) (width 0.2) (layer "F.Cu") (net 9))
 (segment (start 62.53 113.67) (end 58.2 113.67) (width 0.2) (layer "F.Cu") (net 9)))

